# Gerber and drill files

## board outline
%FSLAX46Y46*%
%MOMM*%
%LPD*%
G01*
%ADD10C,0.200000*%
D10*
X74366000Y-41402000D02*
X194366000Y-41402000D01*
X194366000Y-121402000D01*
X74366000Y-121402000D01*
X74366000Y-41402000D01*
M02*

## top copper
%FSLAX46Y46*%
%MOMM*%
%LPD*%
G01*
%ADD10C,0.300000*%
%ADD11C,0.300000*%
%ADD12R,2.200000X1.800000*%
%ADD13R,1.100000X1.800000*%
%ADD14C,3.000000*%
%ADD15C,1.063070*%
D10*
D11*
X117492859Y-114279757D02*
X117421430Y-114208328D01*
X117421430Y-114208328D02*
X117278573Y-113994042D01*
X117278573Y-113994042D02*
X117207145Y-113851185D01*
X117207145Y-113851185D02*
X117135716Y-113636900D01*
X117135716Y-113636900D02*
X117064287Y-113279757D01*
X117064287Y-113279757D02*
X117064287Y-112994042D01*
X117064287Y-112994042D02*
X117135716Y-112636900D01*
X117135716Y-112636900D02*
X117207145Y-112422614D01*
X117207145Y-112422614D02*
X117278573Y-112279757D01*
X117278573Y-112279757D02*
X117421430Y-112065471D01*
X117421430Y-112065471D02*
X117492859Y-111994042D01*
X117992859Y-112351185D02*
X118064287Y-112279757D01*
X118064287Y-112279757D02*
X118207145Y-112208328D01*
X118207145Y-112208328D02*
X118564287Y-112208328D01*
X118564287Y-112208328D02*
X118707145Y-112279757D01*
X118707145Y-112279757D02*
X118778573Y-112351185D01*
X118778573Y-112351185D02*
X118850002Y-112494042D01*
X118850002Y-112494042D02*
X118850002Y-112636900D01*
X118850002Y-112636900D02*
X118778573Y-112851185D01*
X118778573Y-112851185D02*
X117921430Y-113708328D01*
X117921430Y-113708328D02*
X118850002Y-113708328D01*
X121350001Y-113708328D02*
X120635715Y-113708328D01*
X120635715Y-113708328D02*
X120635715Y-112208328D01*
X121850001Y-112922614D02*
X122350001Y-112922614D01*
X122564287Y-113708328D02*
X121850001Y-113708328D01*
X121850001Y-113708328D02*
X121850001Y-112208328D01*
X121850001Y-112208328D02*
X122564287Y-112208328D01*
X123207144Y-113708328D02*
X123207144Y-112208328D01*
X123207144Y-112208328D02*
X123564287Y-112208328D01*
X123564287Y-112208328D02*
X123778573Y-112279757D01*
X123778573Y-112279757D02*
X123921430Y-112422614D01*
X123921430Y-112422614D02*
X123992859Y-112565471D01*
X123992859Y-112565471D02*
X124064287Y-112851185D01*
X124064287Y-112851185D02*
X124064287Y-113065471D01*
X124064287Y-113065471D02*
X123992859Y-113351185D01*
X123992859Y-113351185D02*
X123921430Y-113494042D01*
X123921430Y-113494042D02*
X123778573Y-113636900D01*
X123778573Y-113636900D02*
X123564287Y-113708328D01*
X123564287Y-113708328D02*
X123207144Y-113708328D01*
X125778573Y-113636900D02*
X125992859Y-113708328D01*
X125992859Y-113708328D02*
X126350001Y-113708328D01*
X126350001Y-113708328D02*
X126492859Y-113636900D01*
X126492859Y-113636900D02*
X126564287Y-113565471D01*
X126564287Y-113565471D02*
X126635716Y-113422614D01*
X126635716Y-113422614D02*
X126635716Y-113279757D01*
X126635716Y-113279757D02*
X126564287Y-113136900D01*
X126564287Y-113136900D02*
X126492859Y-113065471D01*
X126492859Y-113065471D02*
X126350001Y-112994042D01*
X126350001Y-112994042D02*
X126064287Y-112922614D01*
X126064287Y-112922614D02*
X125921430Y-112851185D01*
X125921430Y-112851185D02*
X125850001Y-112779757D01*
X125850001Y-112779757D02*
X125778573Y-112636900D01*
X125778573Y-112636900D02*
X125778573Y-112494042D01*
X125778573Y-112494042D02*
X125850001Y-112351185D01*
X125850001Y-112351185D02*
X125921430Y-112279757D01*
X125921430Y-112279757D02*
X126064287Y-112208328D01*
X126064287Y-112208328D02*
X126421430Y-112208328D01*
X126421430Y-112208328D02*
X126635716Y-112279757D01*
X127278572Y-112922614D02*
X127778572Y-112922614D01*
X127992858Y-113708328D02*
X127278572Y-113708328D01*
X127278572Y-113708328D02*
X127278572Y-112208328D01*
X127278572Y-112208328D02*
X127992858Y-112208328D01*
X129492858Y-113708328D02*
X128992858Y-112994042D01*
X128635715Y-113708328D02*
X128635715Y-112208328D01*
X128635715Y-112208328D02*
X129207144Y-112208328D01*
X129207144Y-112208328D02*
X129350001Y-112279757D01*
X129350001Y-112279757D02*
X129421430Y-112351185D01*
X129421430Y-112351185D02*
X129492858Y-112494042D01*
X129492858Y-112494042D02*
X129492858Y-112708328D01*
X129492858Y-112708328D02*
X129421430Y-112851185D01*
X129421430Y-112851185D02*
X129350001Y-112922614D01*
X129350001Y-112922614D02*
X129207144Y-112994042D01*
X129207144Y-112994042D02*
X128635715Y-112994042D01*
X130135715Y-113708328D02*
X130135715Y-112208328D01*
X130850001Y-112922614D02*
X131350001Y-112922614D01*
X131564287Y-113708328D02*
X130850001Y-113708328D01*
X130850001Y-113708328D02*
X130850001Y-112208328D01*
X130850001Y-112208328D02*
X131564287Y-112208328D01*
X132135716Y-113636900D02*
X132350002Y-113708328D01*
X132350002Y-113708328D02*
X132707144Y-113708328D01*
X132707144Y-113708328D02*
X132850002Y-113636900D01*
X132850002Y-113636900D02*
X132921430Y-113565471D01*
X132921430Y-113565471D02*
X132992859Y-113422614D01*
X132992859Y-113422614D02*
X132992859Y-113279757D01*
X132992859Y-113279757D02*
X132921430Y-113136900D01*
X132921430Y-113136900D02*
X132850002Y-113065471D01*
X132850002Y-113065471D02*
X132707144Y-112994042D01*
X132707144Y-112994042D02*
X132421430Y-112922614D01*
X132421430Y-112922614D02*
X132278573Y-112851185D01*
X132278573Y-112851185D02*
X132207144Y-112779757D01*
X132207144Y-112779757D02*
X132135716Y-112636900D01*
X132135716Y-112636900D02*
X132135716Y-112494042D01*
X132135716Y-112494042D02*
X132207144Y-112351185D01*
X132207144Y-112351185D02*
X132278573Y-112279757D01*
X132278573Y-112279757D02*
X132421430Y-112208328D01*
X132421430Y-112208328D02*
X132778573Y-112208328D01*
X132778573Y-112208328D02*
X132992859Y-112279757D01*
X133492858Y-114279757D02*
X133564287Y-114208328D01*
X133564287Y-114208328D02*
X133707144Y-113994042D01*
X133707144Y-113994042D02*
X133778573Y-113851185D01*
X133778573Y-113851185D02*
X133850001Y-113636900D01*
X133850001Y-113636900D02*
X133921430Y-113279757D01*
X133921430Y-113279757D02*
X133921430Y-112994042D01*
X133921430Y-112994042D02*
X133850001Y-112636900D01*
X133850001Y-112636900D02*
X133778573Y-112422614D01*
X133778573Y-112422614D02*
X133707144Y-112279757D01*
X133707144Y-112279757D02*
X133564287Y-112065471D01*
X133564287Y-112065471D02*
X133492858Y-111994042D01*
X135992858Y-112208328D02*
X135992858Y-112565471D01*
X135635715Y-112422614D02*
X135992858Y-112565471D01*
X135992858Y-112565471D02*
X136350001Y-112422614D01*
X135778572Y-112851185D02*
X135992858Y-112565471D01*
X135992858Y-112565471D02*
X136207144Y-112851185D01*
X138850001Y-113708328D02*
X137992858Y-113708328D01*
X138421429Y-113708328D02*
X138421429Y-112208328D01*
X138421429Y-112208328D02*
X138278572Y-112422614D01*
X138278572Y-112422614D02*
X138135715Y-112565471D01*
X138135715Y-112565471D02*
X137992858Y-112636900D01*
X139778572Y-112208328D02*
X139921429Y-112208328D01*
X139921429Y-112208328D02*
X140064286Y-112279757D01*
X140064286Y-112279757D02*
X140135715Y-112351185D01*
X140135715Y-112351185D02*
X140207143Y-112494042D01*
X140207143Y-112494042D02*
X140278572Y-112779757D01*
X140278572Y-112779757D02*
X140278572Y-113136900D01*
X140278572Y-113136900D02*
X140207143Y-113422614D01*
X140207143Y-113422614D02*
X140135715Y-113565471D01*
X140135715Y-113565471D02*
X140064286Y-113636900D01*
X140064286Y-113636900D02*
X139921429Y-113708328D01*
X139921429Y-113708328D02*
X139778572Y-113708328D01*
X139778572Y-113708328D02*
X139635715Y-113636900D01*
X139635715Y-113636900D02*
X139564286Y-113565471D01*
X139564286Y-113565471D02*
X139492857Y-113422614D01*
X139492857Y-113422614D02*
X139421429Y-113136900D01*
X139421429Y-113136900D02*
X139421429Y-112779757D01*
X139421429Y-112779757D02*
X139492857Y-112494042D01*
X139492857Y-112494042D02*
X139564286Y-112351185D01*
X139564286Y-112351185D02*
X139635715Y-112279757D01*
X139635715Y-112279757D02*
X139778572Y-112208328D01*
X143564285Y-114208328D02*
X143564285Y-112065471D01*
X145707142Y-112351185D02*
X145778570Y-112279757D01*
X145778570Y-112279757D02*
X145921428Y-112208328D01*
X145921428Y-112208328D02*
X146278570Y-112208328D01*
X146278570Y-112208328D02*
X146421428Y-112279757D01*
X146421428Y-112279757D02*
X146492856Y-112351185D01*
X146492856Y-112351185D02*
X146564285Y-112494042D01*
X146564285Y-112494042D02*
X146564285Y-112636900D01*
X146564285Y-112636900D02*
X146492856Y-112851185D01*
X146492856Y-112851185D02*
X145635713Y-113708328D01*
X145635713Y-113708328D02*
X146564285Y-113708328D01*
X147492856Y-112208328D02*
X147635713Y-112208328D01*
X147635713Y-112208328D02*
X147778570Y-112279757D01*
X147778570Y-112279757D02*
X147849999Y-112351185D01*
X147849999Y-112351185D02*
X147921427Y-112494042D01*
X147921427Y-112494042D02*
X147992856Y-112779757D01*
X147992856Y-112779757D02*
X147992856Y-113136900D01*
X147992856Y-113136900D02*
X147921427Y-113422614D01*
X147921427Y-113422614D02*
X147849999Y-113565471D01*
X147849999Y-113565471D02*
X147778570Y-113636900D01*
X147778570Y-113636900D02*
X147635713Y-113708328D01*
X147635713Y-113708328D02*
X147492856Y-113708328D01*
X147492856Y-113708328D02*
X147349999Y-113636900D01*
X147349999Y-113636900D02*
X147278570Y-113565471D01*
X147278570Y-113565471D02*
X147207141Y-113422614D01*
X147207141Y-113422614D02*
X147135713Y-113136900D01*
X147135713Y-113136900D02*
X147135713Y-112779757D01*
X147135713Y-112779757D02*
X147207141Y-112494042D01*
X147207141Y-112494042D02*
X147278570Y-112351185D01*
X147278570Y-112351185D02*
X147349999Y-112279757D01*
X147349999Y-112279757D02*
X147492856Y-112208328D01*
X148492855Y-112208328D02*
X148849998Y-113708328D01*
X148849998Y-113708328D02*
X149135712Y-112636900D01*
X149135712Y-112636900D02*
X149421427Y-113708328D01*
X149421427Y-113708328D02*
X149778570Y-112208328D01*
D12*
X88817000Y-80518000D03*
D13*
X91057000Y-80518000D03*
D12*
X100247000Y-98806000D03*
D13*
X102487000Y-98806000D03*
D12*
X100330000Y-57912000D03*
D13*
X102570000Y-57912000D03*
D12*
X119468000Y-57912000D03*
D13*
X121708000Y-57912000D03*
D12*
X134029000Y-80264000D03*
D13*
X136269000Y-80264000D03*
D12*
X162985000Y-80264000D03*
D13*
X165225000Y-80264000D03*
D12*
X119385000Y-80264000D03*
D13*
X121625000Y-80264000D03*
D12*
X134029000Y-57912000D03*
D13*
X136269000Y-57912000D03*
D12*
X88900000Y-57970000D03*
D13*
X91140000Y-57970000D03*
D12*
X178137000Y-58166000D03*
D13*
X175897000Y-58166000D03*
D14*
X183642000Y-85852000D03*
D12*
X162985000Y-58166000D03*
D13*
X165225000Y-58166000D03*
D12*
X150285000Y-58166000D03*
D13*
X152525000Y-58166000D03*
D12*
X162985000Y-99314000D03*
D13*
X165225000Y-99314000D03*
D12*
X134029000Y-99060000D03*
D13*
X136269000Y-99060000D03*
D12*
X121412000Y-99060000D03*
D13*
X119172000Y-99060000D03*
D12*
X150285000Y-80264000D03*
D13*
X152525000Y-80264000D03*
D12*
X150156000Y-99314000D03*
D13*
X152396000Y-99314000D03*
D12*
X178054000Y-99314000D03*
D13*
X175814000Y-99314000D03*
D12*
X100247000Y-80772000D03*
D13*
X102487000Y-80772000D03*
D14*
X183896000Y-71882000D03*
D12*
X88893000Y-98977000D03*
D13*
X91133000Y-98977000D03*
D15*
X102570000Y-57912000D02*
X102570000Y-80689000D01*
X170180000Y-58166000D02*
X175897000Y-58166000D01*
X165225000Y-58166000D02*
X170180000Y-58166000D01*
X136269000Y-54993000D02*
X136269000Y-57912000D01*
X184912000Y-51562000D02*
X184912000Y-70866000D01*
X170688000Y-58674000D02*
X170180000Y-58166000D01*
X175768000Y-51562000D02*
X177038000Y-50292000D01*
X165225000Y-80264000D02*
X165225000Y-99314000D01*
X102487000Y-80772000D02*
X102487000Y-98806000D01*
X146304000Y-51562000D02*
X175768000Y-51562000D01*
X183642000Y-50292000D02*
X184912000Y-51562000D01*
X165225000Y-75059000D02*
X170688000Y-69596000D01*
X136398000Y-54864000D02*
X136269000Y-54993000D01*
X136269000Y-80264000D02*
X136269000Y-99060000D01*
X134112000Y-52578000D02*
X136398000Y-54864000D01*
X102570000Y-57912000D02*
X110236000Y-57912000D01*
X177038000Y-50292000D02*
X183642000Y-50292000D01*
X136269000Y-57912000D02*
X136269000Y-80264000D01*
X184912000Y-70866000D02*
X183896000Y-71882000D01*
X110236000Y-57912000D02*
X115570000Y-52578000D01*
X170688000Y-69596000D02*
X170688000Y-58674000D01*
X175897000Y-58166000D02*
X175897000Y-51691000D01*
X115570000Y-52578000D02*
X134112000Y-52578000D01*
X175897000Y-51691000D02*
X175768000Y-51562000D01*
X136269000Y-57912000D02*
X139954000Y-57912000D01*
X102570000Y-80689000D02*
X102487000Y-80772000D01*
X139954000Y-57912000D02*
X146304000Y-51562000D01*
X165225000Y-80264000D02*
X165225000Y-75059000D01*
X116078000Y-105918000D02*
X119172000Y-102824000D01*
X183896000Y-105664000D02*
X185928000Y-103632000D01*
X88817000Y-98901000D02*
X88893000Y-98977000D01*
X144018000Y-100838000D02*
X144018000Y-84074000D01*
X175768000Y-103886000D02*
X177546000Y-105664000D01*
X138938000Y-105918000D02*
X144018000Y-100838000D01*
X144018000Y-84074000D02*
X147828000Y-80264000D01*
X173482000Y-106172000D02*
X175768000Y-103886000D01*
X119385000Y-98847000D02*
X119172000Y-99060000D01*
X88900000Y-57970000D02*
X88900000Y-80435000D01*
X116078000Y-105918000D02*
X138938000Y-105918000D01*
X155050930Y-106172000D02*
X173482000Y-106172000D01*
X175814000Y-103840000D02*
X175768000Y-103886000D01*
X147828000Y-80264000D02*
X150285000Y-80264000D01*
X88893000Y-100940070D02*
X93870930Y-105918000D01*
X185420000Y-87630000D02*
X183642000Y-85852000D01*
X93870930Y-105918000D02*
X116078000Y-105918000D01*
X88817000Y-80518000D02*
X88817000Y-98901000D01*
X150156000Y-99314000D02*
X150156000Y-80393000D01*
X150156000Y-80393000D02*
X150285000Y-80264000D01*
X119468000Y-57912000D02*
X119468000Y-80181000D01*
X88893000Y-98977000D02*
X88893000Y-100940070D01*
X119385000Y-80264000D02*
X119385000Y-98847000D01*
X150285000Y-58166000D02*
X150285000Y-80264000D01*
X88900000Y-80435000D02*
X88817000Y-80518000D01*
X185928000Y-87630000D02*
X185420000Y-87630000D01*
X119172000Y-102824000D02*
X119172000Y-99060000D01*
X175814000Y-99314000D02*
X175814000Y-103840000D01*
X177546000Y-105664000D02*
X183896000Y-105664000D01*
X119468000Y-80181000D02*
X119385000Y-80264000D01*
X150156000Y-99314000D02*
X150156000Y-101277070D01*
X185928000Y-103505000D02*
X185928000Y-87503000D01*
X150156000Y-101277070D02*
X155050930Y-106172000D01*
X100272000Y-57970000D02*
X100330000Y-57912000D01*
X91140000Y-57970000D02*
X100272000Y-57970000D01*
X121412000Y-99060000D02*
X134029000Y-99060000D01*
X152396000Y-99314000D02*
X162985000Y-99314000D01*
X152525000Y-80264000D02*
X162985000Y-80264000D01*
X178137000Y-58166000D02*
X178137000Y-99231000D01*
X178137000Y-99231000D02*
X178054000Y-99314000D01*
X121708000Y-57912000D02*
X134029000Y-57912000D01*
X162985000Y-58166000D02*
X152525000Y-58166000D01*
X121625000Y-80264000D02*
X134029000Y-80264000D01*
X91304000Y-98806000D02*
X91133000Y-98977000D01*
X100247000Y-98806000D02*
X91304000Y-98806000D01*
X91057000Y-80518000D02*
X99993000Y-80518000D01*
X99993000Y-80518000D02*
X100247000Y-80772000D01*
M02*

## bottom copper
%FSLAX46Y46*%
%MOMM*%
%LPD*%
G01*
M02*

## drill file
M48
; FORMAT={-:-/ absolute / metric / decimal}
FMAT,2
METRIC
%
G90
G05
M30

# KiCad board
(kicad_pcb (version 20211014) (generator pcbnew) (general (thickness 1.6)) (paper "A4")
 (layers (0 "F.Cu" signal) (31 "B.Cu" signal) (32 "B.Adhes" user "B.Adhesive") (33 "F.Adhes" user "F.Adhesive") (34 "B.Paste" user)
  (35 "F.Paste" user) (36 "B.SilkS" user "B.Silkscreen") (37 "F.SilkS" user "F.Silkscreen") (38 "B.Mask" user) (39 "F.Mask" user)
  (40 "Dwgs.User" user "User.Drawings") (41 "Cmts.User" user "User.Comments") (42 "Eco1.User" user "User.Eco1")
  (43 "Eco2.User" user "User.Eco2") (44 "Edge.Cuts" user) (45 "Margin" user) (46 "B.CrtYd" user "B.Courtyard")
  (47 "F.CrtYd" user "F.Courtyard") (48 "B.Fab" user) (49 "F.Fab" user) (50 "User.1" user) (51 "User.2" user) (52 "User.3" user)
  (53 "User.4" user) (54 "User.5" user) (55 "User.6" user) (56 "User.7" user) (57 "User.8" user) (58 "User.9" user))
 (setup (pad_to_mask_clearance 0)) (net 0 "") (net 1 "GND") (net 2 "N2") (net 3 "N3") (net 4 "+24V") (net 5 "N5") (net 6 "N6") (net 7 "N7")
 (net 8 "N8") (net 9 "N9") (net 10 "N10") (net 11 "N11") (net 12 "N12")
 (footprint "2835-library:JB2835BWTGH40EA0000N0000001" (layer "F.Cu") (at 88.817 80.518)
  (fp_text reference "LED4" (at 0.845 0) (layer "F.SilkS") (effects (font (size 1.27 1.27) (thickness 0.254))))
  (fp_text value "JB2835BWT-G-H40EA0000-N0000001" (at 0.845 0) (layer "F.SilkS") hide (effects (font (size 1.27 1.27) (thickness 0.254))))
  (pad "1" smd rect locked (at 0 0 90) (size 1.8 2.2) (layers "F.Cu" "F.Paste" "F.Mask") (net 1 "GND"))
  (pad "2" smd rect locked (at 2.24 0) (size 1.1 1.8) (layers "F.Cu" "F.Paste" "F.Mask") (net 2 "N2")))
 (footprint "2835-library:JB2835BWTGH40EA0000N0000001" (layer "F.Cu") (at 100.247 98.806)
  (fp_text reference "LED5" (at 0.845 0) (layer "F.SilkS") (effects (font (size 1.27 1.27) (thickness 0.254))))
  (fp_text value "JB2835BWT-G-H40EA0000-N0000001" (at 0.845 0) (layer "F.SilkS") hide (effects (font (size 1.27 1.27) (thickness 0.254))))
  (pad "1" smd rect locked (at 0 0 90) (size 1.8 2.2) (layers "F.Cu" "F.Paste" "F.Mask") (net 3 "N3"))
  (pad "2" smd rect locked (at 2.24 0) (size 1.1 1.8) (layers "F.Cu" "F.Paste" "F.Mask") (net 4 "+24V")))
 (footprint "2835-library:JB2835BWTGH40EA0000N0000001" (layer "F.Cu") (at 100.33 57.912)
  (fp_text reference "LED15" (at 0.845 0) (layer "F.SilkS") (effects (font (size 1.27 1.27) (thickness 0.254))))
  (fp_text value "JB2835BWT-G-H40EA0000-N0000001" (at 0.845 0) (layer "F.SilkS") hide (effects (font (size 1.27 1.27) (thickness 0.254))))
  (pad "1" smd rect locked (at 0 0 90) (size 1.8 2.2) (layers "F.Cu" "F.Paste" "F.Mask") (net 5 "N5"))
  (pad "2" smd rect locked (at 2.24 0) (size 1.1 1.8) (layers "F.Cu" "F.Paste" "F.Mask") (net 4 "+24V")))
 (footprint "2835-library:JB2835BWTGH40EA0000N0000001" (layer "F.Cu") (at 119.468 57.912)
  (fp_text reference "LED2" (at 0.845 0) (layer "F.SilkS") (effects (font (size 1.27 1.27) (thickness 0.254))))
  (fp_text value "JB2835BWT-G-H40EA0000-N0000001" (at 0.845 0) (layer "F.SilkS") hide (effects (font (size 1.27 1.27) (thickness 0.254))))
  (pad "1" smd rect locked (at 0 0 90) (size 1.8 2.2) (layers "F.Cu" "F.Paste" "F.Mask") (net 1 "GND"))
  (pad "2" smd rect locked (at 2.24 0) (size 1.1 1.8) (layers "F.Cu" "F.Paste" "F.Mask") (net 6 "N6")))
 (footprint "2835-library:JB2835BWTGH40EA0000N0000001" (layer "F.Cu") (at 134.029 80.264)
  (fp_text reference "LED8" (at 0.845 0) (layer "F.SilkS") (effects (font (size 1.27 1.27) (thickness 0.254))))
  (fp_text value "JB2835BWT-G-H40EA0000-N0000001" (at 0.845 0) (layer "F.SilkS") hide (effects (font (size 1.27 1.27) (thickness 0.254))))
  (pad "1" smd rect locked (at 0 0 90) (size 1.8 2.2) (layers "F.Cu" "F.Paste" "F.Mask") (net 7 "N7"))
  (pad "2" smd rect locked (at 2.24 0) (size 1.1 1.8) (layers "F.Cu" "F.Paste" "F.Mask") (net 4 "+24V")))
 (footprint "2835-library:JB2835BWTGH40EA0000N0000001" (layer "F.Cu") (at 162.985 80.264)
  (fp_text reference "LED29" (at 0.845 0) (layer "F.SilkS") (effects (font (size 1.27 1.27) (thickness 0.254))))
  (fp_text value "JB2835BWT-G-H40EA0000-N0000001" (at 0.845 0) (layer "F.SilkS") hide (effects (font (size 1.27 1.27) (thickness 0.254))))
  (pad "1" smd rect locked (at 0 0 90) (size 1.8 2.2) (layers "F.Cu" "F.Paste" "F.Mask") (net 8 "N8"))
  (pad "2" smd rect locked (at 2.24 0) (size 1.1 1.8) (layers "F.Cu" "F.Paste" "F.Mask") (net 4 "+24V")))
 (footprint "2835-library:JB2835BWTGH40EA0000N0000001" (layer "F.Cu") (at 119.385 80.264)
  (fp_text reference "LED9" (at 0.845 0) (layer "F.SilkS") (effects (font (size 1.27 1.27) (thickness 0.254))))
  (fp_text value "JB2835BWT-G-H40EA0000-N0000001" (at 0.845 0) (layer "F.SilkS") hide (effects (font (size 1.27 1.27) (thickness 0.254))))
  (pad "1" smd rect locked (at 0 0 90) (size 1.8 2.2) (layers "F.Cu" "F.Paste" "F.Mask") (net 1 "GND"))
  (pad "2" smd rect locked (at 2.24 0) (size 1.1 1.8) (layers "F.Cu" "F.Paste" "F.Mask") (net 7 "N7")))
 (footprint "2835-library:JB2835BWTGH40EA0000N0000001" (layer "F.Cu") (at 134.029 57.912)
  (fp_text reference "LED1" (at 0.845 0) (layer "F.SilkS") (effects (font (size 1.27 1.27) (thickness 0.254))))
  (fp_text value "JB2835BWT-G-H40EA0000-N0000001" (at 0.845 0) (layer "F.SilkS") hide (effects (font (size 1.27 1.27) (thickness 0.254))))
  (pad "1" smd rect locked (at 0 0 90) (size 1.8 2.2) (layers "F.Cu" "F.Paste" "F.Mask") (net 6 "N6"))
  (pad "2" smd rect locked (at 2.24 0) (size 1.1 1.8) (layers "F.Cu" "F.Paste" "F.Mask") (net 4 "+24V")))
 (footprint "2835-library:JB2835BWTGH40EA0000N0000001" (layer "F.Cu") (at 88.9 57.97)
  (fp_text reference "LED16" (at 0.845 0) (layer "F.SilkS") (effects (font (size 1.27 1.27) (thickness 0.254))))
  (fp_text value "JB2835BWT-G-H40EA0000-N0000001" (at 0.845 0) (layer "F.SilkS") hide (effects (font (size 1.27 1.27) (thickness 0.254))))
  (pad "1" smd rect locked (at 0 0 90) (size 1.8 2.2) (layers "F.Cu" "F.Paste" "F.Mask") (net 1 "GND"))
  (pad "2" smd rect locked (at 2.24 0) (size 1.1 1.8) (layers "F.Cu" "F.Paste" "F.Mask") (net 5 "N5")))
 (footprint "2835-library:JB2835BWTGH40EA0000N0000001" (layer "F.Cu") (at 178.137 58.166 180)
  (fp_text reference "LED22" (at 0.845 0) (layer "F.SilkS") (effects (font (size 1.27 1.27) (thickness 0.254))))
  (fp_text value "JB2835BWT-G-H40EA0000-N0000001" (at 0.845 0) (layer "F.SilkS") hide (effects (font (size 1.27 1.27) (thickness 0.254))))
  (pad "1" smd rect locked (at 0 0 270) (size 1.8 2.2) (layers "F.Cu" "F.Paste" "F.Mask") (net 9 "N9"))
  (pad "2" smd rect locked (at 2.24 0 180) (size 1.1 1.8) (layers "F.Cu" "F.Paste" "F.Mask") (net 4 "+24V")))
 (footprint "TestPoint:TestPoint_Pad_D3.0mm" (layer "F.Cu") (at 183.642 85.852)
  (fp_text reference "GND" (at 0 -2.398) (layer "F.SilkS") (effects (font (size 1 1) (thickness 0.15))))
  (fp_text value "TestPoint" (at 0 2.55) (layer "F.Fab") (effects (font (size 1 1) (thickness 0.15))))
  (pad "1" smd circle (at 0 0) (size 3 3) (layers "F.Cu" "F.Mask") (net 1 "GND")))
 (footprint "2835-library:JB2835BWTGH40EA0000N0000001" (layer "F.Cu") (at 162.985 58.166)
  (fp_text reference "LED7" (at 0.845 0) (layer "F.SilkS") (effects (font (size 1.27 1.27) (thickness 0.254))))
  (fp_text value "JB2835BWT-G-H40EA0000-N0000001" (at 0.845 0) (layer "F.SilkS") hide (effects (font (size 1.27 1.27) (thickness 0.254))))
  (pad "1" smd rect locked (at 0 0 90) (size 1.8 2.2) (layers "F.Cu" "F.Paste" "F.Mask") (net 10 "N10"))
  (pad "2" smd rect locked (at 2.24 0) (size 1.1 1.8) (layers "F.Cu" "F.Paste" "F.Mask") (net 4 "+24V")))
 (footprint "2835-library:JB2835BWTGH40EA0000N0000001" (layer "F.Cu") (at 150.285 58.166)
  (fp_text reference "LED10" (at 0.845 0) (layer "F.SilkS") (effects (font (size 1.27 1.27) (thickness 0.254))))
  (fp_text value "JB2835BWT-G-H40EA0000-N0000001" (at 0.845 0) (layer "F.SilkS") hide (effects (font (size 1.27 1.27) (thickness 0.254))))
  (pad "1" smd rect locked (at 0 0 90) (size 1.8 2.2) (layers "F.Cu" "F.Paste" "F.Mask") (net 1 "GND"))
  (pad "2" smd rect locked (at 2.24 0) (size 1.1 1.8) (layers "F.Cu" "F.Paste" "F.Mask") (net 10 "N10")))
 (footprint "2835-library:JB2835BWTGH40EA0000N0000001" (layer "F.Cu") (at 162.985 99.314)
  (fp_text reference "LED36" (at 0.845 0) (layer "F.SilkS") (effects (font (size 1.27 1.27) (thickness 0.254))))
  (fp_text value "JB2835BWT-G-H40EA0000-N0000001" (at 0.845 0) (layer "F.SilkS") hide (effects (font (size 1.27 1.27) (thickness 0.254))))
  (pad "1" smd rect locked (at 0 0 90) (size 1.8 2.2) (layers "F.Cu" "F.Paste" "F.Mask") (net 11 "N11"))
  (pad "2" smd rect locked (at 2.24 0) (size 1.1 1.8) (layers "F.Cu" "F.Paste" "F.Mask") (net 4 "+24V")))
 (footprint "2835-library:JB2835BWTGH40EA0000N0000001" (layer "F.Cu") (at 134.029 99.06)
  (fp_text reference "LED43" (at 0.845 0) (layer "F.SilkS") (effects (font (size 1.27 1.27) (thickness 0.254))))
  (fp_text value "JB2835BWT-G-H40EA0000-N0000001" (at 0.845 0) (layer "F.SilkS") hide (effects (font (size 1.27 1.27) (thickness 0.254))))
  (pad "1" smd rect locked (at 0 0 90) (size 1.8 2.2) (layers "F.Cu" "F.Paste" "F.Mask") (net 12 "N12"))
  (pad "2" smd rect locked (at 2.24 0) (size 1.1 1.8) (layers "F.Cu" "F.Paste" "F.Mask") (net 4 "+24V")))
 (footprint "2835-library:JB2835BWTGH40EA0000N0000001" (layer "F.Cu") (at 121.412 99.06 180)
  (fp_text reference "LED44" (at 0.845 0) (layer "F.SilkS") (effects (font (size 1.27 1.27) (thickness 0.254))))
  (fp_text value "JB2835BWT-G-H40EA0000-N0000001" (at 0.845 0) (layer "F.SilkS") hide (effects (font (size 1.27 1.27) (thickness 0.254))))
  (pad "1" smd rect locked (at 0 0 270) (size 1.8 2.2) (layers "F.Cu" "F.Paste" "F.Mask") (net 12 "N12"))
  (pad "2" smd rect locked (at 2.24 0 180) (size 1.1 1.8) (layers "F.Cu" "F.Paste" "F.Mask") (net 1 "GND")))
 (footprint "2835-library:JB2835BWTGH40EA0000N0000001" (layer "F.Cu") (at 150.285 80.264)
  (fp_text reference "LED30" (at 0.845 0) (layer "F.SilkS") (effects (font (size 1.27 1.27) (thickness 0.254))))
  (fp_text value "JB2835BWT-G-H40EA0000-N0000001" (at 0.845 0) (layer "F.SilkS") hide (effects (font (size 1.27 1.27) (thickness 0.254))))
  (pad "1" smd rect locked (at 0 0 90) (size 1.8 2.2) (layers "F.Cu" "F.Paste" "F.Mask") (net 1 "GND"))
  (pad "2" smd rect locked (at 2.24 0) (size 1.1 1.8) (layers "F.Cu" "F.Paste" "F.Mask") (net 8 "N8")))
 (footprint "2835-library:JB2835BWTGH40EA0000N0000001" (layer "F.Cu") (at 150.156 99.314)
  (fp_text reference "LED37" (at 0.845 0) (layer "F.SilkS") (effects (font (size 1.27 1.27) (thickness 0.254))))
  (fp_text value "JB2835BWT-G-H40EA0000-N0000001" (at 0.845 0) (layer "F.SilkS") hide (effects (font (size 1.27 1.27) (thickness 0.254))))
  (pad "1" smd rect locked (at 0 0 90) (size 1.8 2.2) (layers "F.Cu" "F.Paste" "F.Mask") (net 1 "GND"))
  (pad "2" smd rect locked (at 2.24 0) (size 1.1 1.8) (layers "F.Cu" "F.Paste" "F.Mask") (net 11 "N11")))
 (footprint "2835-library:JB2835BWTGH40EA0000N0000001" (layer "F.Cu") (at 178.054 99.314 180)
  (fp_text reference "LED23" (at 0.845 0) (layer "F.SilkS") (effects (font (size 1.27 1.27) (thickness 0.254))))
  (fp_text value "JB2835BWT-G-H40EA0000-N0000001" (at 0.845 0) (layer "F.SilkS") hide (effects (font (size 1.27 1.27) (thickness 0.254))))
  (pad "1" smd rect locked (at 0 0 270) (size 1.8 2.2) (layers "F.Cu" "F.Paste" "F.Mask") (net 9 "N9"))
  (pad "2" smd rect locked (at 2.24 0 180) (size 1.1 1.8) (layers "F.Cu" "F.Paste" "F.Mask") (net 1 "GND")))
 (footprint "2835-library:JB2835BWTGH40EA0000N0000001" (layer "F.Cu") (at 100.247 80.772)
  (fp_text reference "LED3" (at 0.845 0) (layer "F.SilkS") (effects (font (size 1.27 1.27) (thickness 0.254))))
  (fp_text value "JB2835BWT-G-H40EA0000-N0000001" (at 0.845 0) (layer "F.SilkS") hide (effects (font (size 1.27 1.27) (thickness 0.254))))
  (pad "1" smd rect locked (at 0 0 90) (size 1.8 2.2) (layers "F.Cu" "F.Paste" "F.Mask") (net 2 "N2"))
  (pad "2" smd rect locked (at 2.24 0) (size 1.1 1.8) (layers "F.Cu" "F.Paste" "F.Mask") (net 4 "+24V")))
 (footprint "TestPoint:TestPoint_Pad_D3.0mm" (layer "F.Cu") (at 183.896 71.882)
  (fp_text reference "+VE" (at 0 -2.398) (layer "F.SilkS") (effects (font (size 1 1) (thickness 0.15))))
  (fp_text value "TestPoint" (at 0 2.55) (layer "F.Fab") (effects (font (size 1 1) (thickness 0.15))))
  (pad "1" smd circle (at 0 0) (size 3 3) (layers "F.Cu" "F.Mask") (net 4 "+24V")))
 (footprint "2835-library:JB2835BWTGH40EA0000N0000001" (layer "F.Cu") (at 88.893 98.977)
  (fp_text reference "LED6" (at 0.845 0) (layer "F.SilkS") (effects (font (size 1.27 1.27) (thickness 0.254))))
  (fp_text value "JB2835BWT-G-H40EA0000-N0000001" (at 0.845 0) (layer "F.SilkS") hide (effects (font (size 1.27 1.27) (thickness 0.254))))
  (pad "1" smd rect locked (at 0 0 90) (size 1.8 2.2) (layers "F.Cu" "F.Paste" "F.Mask") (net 1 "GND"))
  (pad "2" smd rect locked (at 2.24 0) (size 1.1 1.8) (layers "F.Cu" "F.Paste" "F.Mask") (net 3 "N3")))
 (gr_rect (start 74.366 41.402) (end 194.366 121.402) (layer "Edge.Cuts") (width 0.2) (fill none))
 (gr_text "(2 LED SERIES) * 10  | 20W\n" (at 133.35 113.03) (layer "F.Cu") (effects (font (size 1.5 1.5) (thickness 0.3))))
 (segment (start 102.57 57.912) (end 102.57 80.689) (width 1.06307) (layer "F.Cu") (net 4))
 (segment (start 170.18 58.166) (end 175.897 58.166) (width 1.06307) (layer "F.Cu") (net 4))
 (segment (start 165.225 58.166) (end 170.18 58.166) (width 1.06307) (layer "F.Cu") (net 4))
 (segment (start 136.269 54.993) (end 136.269 57.912) (width 1.06307) (layer "F.Cu") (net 4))
 (segment (start 184.912 51.562) (end 184.912 70.866) (width 1.06307) (layer "F.Cu") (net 4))
 (segment (start 170.688 58.674) (end 170.18 58.166) (width 1.06307) (layer "F.Cu") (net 4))
 (segment (start 175.768 51.562) (end 177.038 50.292) (width 1.06307) (layer "F.Cu") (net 4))
 (segment (start 165.225 80.264) (end 165.225 99.314) (width 1.06307) (layer "F.Cu") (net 4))
 (segment (start 102.487 80.772) (end 102.487 98.806) (width 1.06307) (layer "F.Cu") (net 4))
 (segment (start 146.304 51.562) (end 175.768 51.562) (width 1.06307) (layer "F.Cu") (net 4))
 (segment (start 183.642 50.292) (end 184.912 51.562) (width 1.06307) (layer "F.Cu") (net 4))
 (segment (start 165.225 75.059) (end 170.688 69.596) (width 1.06307) (layer "F.Cu") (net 4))
 (segment (start 136.398 54.864) (end 136.269 54.993) (width 1.06307) (layer "F.Cu") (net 4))
 (segment (start 136.269 80.264) (end 136.269 99.06) (width 1.06307) (layer "F.Cu") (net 4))
 (segment (start 134.112 52.578) (end 136.398 54.864) (width 1.06307) (layer "F.Cu") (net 4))
 (segment (start 102.57 57.912) (end 110.236 57.912) (width 1.06307) (layer "F.Cu") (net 4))
 (segment (start 177.038 50.292) (end 183.642 50.292) (width 1.06307) (layer "F.Cu") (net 4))
 (segment (start 136.269 57.912) (end 136.269 80.264) (width 1.06307) (layer "F.Cu") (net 4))
 (segment (start 184.912 70.866) (end 183.896 71.882) (width 1.06307) (layer "F.Cu") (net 4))
 (segment (start 110.236 57.912) (end 115.57 52.578) (width 1.06307) (layer "F.Cu") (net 4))
 (segment (start 170.688 69.596) (end 170.688 58.674) (width 1.06307) (layer "F.Cu") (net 4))
 (segment (start 175.897 58.166) (end 175.897 51.691) (width 1.06307) (layer "F.Cu") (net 4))
 (segment (start 115.57 52.578) (end 134.112 52.578) (width 1.06307) (layer "F.Cu") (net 4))
 (segment (start 175.897 51.691) (end 175.768 51.562) (width 1.06307) (layer "F.Cu") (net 4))
 (segment (start 136.269 57.912) (end 139.954 57.912) (width 1.06307) (layer "F.Cu") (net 4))
 (segment (start 102.57 80.689) (end 102.487 80.772) (width 1.06307) (layer "F.Cu") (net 4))
 (segment (start 139.954 57.912) (end 146.304 51.562) (width 1.06307) (layer "F.Cu") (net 4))
 (segment (start 165.225 80.264) (end 165.225 75.059) (width 1.06307) (layer "F.Cu") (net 4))
 (segment (start 116.078 105.918) (end 119.172 102.824) (width 1.06307) (layer "F.Cu") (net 1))
 (segment (start 183.896 105.664) (end 185.928 103.632) (width 1.06307) (layer "F.Cu") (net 1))
 (segment (start 88.817 98.901) (end 88.893 98.977) (width 1.06307) (layer "F.Cu") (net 1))
 (segment (start 144.018 100.838) (end 144.018 84.074) (width 1.06307) (layer "F.Cu") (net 1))
 (segment (start 175.768 103.886) (end 177.546 105.664) (width 1.06307) (layer "F.Cu") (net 1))
 (segment (start 138.938 105.918) (end 144.018 100.838) (width 1.06307) (layer "F.Cu") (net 1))
 (segment (start 144.018 84.074) (end 147.828 80.264) (width 1.06307) (layer "F.Cu") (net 1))
 (segment (start 173.482 106.172) (end 175.768 103.886) (width 1.06307) (layer "F.Cu") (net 1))
 (segment (start 119.385 98.847) (end 119.172 99.06) (width 1.06307) (layer "F.Cu") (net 1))
 (segment (start 88.9 57.97) (end 88.9 80.435) (width 1.06307) (layer "F.Cu") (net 1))
 (segment (start 116.078 105.918) (end 138.938 105.918) (width 1.06307) (layer "F.Cu") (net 1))
 (segment (start 155.05093 106.172) (end 173.482 106.172) (width 1.06307) (layer "F.Cu") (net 1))
 (segment (start 175.814 103.84) (end 175.768 103.886) (width 1.06307) (layer "F.Cu") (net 1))
 (segment (start 147.828 80.264) (end 150.285 80.264) (width 1.06307) (layer "F.Cu") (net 1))
 (segment (start 88.893 100.94007) (end 93.87093 105.918) (width 1.06307) (layer "F.Cu") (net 1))
 (segment (start 185.42 87.63) (end 183.642 85.852) (width 1.06307) (layer "F.Cu") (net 1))
 (segment (start 93.87093 105.918) (end 116.078 105.918) (width 1.06307) (layer "F.Cu") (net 1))
 (segment (start 88.817 80.518) (end 88.817 98.901) (width 1.06307) (layer "F.Cu") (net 1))
 (segment (start 150.156 99.314) (end 150.156 80.393) (width 1.06307) (layer "F.Cu") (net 1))
 (segment (start 150.156 80.393) (end 150.285 80.264) (width 1.06307) (layer "F.Cu") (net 1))
 (segment (start 119.468 57.912) (end 119.468 80.181) (width 1.06307) (layer "F.Cu") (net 1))
 (segment (start 88.893 98.977) (end 88.893 100.94007) (width 1.06307) (layer "F.Cu") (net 1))
 (segment (start 119.385 80.264) (end 119.385 98.847) (width 1.06307) (layer "F.Cu") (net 1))
 (segment (start 150.285 58.166) (end 150.285 80.264) (width 1.06307) (layer "F.Cu") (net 1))
 (segment (start 88.9 80.435) (end 88.817 80.518) (width 1.06307) (layer "F.Cu") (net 1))
 (segment (start 185.928 87.63) (end 185.42 87.63) (width 1.06307) (layer "F.Cu") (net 1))
 (segment (start 119.172 102.824) (end 119.172 99.06) (width 1.06307) (layer "F.Cu") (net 1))
 (segment (start 175.814 99.314) (end 175.814 103.84) (width 1.06307) (layer "F.Cu") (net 1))
 (segment (start 177.546 105.664) (end 183.896 105.664) (width 1.06307) (layer "F.Cu") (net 1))
 (segment (start 119.468 80.181) (end 119.385 80.264) (width 1.06307) (layer "F.Cu") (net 1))
 (segment (start 150.156 99.314) (end 150.156 101.27707) (width 1.06307) (layer "F.Cu") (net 1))
 (segment (start 185.928 103.505) (end 185.928 87.503) (width 1.06307) (layer "F.Cu") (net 1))
 (segment (start 150.156 101.27707) (end 155.05093 106.172) (width 1.06307) (layer "F.Cu") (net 1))
 (segment (start 100.272 57.97) (end 100.33 57.912) (width 1.06307) (layer "F.Cu") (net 5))
 (segment (start 91.14 57.97) (end 100.272 57.97) (width 1.06307) (layer "F.Cu") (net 5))
 (segment (start 121.412 99.06) (end 134.029 99.06) (width 1.06307) (layer "F.Cu") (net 12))
 (segment (start 152.396 99.314) (end 162.985 99.314) (width 1.06307) (layer "F.Cu") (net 11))
 (segment (start 152.525 80.264) (end 162.985 80.264) (width 1.06307) (layer "F.Cu") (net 8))
 (segment (start 178.137 58.166) (end 178.137 99.231) (width 1.06307) (layer "F.Cu") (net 9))
 (segment (start 178.137 99.231) (end 178.054 99.314) (width 1.06307) (layer "F.Cu") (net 9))
 (segment (start 121.708 57.912) (end 134.029 57.912) (width 1.06307) (layer "F.Cu") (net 6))
 (segment (start 162.985 58.166) (end 152.525 58.166) (width 1.06307) (layer "F.Cu") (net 10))
 (segment (start 121.625 80.264) (end 134.029 80.264) (width 1.06307) (layer "F.Cu") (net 7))
 (segment (start 91.304 98.806) (end 91.133 98.977) (width 1.06307) (layer "F.Cu") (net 3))
 (segment (start 100.247 98.806) (end 91.304 98.806) (width 1.06307) (layer "F.Cu") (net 3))
 (segment (start 91.057 80.518) (end 99.993 80.518) (width 1.06307) (layer "F.Cu") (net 2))
 (segment (start 99.993 80.518) (end 100.247 80.772) (width 1.06307) (layer "F.Cu") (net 2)))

